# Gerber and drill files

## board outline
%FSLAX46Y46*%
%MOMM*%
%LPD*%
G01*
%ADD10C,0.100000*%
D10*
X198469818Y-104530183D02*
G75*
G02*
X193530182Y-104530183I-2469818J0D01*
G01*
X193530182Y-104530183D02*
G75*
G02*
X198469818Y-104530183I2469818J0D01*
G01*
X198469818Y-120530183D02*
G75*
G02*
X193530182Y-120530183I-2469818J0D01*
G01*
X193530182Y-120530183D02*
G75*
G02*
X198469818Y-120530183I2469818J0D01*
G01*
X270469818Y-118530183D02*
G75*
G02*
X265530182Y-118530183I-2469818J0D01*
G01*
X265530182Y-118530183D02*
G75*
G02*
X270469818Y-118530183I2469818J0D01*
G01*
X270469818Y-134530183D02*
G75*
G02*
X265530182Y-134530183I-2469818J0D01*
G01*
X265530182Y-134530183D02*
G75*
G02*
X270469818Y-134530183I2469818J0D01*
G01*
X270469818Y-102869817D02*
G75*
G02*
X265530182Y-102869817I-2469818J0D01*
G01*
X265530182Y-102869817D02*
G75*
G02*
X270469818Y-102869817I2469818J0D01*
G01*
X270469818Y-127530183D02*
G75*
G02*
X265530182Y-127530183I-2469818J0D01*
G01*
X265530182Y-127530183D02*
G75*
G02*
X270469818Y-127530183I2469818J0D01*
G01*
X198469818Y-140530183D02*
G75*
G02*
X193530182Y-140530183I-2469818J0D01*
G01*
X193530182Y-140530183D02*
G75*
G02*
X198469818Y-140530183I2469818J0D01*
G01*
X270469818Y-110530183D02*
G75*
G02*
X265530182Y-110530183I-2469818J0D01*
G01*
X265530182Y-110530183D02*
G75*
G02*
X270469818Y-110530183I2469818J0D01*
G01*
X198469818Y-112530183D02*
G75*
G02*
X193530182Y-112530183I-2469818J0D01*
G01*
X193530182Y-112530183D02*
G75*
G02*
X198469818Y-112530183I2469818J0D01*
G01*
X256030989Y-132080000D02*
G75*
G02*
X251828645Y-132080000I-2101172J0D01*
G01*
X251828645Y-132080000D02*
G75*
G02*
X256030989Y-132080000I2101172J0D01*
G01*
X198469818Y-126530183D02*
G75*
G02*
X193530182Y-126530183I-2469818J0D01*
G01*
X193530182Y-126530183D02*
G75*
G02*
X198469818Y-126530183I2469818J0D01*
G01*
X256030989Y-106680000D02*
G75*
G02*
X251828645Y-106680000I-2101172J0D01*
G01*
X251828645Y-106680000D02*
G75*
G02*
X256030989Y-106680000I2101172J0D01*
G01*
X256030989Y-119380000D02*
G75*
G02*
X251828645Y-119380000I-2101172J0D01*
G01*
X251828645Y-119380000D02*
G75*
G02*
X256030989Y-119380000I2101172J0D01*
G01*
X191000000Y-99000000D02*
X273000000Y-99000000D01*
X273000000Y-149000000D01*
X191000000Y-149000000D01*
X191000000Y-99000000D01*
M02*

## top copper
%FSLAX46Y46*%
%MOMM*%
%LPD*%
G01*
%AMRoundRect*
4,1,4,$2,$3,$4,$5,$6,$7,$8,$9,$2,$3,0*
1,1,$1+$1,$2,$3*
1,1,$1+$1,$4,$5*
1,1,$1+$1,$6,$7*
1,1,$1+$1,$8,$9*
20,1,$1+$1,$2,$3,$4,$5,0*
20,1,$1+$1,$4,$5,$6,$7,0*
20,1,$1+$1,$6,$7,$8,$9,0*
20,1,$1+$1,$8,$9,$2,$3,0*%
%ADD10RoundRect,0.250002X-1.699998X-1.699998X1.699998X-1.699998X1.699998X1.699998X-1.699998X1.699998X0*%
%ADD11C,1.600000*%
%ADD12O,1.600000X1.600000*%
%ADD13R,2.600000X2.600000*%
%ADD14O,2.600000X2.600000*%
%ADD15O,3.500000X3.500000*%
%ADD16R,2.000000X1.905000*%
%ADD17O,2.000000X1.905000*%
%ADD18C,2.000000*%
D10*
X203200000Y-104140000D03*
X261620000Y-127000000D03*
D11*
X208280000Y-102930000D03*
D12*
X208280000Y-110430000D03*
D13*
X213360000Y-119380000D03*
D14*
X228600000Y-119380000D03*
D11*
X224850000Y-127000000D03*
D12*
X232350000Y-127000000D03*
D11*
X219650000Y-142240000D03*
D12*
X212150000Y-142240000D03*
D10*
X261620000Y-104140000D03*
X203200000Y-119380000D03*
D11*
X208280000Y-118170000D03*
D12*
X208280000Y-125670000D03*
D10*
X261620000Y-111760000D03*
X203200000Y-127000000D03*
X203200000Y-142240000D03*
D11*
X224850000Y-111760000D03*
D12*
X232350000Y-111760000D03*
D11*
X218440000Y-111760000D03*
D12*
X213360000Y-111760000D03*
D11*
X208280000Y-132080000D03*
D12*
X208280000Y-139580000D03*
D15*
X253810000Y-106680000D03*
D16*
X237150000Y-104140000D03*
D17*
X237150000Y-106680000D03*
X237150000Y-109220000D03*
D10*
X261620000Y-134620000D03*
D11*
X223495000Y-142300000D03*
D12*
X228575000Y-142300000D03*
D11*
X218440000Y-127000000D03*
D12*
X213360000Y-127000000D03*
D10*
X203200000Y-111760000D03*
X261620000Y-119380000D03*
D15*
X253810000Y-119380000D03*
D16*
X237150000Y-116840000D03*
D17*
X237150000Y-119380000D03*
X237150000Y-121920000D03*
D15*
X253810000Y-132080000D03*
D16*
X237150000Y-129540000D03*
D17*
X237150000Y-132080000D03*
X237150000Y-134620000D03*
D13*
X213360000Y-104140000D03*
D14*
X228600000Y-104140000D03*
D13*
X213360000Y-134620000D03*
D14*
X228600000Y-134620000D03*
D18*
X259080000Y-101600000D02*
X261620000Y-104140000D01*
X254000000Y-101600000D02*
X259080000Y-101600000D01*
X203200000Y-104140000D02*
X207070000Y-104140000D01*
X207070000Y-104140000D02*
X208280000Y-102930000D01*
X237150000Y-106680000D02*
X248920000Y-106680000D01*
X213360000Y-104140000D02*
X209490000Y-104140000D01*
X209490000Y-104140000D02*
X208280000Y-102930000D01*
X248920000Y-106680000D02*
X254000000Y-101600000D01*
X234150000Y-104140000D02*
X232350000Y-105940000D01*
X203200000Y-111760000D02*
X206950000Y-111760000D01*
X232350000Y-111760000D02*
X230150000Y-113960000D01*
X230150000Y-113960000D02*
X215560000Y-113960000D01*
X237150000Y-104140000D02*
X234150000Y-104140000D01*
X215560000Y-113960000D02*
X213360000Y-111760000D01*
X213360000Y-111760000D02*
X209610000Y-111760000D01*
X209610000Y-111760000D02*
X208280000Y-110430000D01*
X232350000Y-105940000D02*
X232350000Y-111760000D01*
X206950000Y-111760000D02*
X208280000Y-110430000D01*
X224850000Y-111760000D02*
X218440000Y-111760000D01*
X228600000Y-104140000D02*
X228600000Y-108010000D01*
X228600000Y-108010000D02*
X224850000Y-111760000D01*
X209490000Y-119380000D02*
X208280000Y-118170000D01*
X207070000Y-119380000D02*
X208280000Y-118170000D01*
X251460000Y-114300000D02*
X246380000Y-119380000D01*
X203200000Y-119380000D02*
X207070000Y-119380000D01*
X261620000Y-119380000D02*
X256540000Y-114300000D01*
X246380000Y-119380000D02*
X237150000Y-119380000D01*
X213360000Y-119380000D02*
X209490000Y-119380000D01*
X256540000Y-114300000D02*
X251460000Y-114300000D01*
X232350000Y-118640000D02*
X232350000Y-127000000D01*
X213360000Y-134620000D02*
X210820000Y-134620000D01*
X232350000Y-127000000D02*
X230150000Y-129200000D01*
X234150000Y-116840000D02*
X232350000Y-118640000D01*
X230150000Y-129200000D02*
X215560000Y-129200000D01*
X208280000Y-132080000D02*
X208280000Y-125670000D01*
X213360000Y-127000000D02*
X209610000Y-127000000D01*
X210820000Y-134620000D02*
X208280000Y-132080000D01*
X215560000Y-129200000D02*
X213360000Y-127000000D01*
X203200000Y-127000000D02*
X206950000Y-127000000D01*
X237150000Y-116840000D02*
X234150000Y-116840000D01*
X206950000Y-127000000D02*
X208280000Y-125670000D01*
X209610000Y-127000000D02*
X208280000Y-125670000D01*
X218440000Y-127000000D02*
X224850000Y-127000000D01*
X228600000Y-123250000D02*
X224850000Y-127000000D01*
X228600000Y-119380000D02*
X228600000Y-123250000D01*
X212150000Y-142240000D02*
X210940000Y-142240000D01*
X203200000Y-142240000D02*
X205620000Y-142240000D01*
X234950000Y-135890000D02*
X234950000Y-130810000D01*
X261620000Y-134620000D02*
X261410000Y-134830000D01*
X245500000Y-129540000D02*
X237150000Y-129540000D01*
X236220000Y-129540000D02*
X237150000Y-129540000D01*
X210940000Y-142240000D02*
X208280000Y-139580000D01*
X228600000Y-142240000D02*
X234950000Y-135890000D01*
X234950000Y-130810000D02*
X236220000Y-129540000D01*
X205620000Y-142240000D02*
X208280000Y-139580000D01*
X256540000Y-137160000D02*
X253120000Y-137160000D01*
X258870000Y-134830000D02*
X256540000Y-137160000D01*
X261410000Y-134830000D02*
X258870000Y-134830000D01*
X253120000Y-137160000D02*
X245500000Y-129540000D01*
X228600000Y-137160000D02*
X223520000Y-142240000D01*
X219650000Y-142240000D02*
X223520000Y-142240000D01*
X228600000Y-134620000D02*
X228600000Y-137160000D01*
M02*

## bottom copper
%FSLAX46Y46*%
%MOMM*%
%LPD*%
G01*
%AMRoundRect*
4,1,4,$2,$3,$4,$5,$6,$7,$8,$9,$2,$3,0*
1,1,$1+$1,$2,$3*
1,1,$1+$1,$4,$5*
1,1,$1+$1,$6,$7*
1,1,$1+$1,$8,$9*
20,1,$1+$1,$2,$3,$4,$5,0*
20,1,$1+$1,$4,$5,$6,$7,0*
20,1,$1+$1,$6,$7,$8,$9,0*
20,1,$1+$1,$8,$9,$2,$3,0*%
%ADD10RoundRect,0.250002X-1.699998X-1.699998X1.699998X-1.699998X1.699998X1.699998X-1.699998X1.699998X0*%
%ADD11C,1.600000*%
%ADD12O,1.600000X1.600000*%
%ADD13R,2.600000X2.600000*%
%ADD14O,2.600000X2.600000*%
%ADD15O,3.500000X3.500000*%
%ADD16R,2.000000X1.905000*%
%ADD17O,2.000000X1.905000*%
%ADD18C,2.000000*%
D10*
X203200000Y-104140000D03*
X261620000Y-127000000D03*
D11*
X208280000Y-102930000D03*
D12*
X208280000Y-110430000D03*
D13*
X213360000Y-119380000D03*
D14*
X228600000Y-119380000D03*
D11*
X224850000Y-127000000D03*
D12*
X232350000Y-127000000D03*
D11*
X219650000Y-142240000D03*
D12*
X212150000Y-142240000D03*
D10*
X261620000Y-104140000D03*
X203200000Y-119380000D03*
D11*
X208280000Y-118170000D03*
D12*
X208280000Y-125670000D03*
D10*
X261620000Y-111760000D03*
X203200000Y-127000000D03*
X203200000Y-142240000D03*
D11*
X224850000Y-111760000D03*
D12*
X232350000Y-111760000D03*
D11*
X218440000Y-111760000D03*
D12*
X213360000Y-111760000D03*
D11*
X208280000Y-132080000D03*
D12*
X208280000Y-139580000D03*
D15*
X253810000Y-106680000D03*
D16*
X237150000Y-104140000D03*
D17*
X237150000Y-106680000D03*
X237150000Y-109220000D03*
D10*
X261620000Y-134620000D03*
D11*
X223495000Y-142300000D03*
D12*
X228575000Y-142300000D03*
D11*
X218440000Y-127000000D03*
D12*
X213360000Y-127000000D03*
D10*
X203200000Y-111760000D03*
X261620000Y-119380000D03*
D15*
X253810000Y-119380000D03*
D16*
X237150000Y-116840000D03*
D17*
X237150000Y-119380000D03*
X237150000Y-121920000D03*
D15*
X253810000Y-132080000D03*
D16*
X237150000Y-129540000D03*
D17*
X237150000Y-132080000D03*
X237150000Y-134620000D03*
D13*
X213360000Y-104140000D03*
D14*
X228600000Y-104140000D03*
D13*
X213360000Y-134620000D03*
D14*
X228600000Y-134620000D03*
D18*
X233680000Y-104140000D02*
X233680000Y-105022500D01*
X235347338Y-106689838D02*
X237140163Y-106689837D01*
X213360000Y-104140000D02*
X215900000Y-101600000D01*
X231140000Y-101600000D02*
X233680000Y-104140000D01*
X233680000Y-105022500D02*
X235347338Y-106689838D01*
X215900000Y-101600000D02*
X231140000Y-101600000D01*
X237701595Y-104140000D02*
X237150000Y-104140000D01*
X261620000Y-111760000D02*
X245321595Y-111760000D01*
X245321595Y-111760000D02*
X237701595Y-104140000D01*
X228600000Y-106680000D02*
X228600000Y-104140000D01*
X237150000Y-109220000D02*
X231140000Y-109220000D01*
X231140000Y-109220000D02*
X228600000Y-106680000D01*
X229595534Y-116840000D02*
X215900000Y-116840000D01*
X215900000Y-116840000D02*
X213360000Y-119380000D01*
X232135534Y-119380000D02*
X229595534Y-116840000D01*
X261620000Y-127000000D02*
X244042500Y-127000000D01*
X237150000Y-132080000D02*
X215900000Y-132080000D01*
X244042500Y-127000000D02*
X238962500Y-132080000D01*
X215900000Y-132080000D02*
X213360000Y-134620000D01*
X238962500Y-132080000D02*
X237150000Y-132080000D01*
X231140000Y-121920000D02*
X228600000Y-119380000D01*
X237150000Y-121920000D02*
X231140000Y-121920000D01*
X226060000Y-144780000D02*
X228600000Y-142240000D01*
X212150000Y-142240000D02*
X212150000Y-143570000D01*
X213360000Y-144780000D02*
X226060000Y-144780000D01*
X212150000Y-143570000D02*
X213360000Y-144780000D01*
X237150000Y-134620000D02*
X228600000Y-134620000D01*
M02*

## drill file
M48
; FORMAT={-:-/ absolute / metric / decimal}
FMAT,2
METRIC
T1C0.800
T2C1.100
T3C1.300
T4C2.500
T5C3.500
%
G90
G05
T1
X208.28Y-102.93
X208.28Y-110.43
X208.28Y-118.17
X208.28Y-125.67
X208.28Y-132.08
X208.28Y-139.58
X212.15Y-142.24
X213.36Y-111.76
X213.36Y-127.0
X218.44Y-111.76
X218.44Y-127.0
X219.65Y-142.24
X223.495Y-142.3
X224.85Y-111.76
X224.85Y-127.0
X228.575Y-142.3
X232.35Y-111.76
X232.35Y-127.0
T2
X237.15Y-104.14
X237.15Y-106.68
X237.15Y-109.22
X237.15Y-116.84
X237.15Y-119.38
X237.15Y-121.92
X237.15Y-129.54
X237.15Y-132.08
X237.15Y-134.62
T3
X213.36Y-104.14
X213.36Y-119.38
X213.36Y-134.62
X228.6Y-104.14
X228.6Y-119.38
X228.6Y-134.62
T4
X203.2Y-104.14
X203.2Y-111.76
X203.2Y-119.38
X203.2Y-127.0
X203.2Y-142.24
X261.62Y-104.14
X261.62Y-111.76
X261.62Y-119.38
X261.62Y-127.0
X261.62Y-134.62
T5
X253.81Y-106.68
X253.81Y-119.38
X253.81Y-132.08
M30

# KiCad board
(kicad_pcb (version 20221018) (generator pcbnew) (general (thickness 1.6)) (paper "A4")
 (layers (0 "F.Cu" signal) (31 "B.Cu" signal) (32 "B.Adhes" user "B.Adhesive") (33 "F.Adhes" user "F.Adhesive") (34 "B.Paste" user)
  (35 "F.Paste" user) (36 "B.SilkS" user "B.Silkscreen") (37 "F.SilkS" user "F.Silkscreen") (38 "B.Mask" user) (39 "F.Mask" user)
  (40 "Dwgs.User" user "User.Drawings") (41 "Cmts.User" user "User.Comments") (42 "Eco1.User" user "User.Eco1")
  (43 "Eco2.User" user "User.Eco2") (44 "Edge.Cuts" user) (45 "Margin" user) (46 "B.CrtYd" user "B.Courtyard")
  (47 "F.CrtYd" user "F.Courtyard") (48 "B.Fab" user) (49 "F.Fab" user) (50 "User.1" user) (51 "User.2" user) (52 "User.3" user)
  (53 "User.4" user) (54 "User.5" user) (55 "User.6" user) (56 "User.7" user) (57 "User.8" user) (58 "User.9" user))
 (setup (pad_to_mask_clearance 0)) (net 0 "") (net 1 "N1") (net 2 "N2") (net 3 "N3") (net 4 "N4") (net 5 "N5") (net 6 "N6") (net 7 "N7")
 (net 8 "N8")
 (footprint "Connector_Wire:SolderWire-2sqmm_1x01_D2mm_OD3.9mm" (layer "F.Cu") (at 203.2 104.14)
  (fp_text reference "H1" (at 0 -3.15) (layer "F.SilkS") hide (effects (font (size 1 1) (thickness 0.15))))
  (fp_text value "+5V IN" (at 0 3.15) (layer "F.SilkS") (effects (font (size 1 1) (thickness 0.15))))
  (pad "1" thru_hole roundrect (at 0 0) (size 3.9 3.9) (drill 2.5) (layers "*.Cu" "*.Mask") (roundrect_rratio 0.06410307692) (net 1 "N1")))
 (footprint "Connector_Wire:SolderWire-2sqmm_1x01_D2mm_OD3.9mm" (layer "F.Cu") (at 261.62 127)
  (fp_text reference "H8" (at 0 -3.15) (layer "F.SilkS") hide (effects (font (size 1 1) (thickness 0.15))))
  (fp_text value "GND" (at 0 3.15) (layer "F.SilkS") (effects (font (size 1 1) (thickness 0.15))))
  (pad "1" thru_hole roundrect (at 0 0) (size 3.9 3.9) (drill 2.5) (layers "*.Cu" "*.Mask") (roundrect_rratio 0.06410307692) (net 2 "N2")))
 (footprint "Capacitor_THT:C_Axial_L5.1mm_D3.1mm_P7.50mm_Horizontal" (layer "F.Cu") (at 208.28 102.93 -90)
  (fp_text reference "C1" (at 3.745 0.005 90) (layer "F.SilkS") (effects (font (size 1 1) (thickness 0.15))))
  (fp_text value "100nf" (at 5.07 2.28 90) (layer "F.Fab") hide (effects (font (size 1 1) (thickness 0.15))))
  (pad "1" thru_hole circle (at 0 0 270) (size 1.6 1.6) (drill 0.8) (layers "*.Cu" "*.Mask") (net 1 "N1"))
  (pad "2" thru_hole oval (at 7.5 0 270) (size 1.6 1.6) (drill 0.8) (layers "*.Cu" "*.Mask") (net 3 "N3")))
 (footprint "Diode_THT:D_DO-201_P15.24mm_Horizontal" (layer "F.Cu") (at 213.36 119.38)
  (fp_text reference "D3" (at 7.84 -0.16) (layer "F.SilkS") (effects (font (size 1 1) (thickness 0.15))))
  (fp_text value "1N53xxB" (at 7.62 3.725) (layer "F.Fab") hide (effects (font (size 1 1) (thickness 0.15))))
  (pad "1" thru_hole rect (at 0 0) (size 2.6 2.6) (drill 1.3) (layers "*.Cu" "*.Mask") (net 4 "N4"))
  (pad "2" thru_hole oval (at 15.24 0) (size 2.6 2.6) (drill 1.3) (layers "*.Cu" "*.Mask") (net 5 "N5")))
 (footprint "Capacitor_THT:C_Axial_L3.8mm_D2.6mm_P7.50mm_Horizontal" (layer "F.Cu") (at 224.85 127)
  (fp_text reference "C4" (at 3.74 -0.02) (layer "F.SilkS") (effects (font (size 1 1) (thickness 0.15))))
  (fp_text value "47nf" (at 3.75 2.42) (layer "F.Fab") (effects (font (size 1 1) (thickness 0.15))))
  (pad "1" thru_hole circle (at 0 0) (size 1.6 1.6) (drill 0.8) (layers "*.Cu" "*.Mask") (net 5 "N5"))
  (pad "2" thru_hole oval (at 7.5 0) (size 1.6 1.6) (drill 0.8) (layers "*.Cu" "*.Mask") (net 2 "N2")))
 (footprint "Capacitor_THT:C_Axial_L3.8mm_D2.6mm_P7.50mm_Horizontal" (layer "F.Cu") (at 219.65 142.24 180)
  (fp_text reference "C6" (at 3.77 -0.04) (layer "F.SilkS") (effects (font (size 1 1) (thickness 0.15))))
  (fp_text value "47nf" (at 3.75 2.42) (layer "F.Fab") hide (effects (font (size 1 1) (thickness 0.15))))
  (pad "1" thru_hole circle (at 0 0 180) (size 1.6 1.6) (drill 0.8) (layers "*.Cu" "*.Mask") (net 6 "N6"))
  (pad "2" thru_hole oval (at 7.5 0 180) (size 1.6 1.6) (drill 0.8) (layers "*.Cu" "*.Mask") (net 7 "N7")))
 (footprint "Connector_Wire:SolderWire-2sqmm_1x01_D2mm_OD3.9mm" (layer "F.Cu") (at 261.62 104.14)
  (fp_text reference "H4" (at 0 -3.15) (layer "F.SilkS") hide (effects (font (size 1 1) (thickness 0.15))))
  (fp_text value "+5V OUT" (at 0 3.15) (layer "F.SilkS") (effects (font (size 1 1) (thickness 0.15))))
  (pad "1" thru_hole roundrect (at 0 0) (size 3.9 3.9) (drill 2.5) (layers "*.Cu" "*.Mask") (roundrect_rratio 0.06410307692) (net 1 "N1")))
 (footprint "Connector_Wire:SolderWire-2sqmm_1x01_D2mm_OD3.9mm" (layer "F.Cu") (at 203.2 119.38)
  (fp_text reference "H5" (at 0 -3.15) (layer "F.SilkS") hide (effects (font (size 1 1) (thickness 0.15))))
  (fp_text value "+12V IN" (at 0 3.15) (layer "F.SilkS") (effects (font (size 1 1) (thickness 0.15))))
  (pad "1" thru_hole roundrect (at 0 0) (size 3.9 3.9) (drill 2.5) (layers "*.Cu" "*.Mask") (roundrect_rratio 0.06410307692) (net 4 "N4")))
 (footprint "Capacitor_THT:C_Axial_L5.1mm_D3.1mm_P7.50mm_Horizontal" (layer "F.Cu") (at 208.28 118.17 -90)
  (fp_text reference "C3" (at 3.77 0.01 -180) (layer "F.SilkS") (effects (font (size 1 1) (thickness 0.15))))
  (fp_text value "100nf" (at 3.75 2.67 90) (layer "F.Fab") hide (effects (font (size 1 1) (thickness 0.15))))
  (pad "1" thru_hole circle (at 0 0 270) (size 1.6 1.6) (drill 0.8) (layers "*.Cu" "*.Mask") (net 4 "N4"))
  (pad "2" thru_hole oval (at 7.5 0 270) (size 1.6 1.6) (drill 0.8) (layers "*.Cu" "*.Mask") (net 2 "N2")))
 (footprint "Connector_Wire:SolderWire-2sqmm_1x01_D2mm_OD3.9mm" (layer "F.Cu") (at 261.62 111.76)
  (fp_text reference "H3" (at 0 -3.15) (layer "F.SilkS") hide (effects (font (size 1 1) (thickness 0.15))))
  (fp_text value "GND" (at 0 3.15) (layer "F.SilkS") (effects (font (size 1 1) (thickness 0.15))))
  (pad "1" thru_hole roundrect (at 0 0) (size 3.9 3.9) (drill 2.5) (layers "*.Cu" "*.Mask") (roundrect_rratio 0.06410307692) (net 3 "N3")))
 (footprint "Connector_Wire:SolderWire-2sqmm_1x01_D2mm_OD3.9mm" (layer "F.Cu") (at 203.2 127)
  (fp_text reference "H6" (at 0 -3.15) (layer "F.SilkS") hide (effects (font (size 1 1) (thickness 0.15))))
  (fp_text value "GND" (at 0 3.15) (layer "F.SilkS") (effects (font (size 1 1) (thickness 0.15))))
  (pad "1" thru_hole roundrect (at 0 0) (size 3.9 3.9) (drill 2.5) (layers "*.Cu" "*.Mask") (roundrect_rratio 0.06410307692) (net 2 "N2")))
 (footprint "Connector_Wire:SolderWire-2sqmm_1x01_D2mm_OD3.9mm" (layer "F.Cu") (at 203.2 142.24)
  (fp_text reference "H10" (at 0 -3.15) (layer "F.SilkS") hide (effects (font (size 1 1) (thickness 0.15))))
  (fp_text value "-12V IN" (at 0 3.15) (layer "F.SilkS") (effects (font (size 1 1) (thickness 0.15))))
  (pad "1" thru_hole roundrect (at 0 0) (size 3.9 3.9) (drill 2.5) (layers "*.Cu" "*.Mask") (roundrect_rratio 0.06410307692) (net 7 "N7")))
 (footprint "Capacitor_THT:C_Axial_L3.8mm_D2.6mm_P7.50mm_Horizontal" (layer "F.Cu") (at 224.85 111.76)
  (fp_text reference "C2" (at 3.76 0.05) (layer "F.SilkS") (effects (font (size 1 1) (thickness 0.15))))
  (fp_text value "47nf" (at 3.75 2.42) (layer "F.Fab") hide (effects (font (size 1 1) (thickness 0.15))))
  (pad "1" thru_hole circle (at 0 0) (size 1.6 1.6) (drill 0.8) (layers "*.Cu" "*.Mask") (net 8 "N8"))
  (pad "2" thru_hole oval (at 7.5 0) (size 1.6 1.6) (drill 0.8) (layers "*.Cu" "*.Mask") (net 3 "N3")))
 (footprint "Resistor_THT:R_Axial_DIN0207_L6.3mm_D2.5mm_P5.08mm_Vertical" (layer "F.Cu") (at 218.44 111.76 180)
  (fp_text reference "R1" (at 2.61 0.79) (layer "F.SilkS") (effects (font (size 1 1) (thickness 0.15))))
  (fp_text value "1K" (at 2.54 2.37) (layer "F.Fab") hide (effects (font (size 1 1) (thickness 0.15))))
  (pad "1" thru_hole circle (at 0 0 180) (size 1.6 1.6) (drill 0.8) (layers "*.Cu" "*.Mask") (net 8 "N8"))
  (pad "2" thru_hole oval (at 5.08 0 180) (size 1.6 1.6) (drill 0.8) (layers "*.Cu" "*.Mask") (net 3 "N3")))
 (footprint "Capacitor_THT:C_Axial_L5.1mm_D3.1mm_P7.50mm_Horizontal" (layer "F.Cu") (at 208.28 132.08 -90)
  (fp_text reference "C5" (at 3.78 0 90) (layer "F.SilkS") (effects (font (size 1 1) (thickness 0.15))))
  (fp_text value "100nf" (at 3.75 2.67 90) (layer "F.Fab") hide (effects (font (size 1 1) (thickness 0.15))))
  (pad "1" thru_hole circle (at 0 0 270) (size 1.6 1.6) (drill 0.8) (layers "*.Cu" "*.Mask") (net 2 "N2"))
  (pad "2" thru_hole oval (at 7.5 0 270) (size 1.6 1.6) (drill 0.8) (layers "*.Cu" "*.Mask") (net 7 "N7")))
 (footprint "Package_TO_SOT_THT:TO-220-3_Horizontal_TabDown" (layer "F.Cu") (at 237.15 104.14 -90)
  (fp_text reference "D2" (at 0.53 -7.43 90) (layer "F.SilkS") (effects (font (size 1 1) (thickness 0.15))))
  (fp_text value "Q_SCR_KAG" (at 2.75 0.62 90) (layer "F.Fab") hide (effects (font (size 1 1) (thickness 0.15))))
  (pad "" thru_hole oval (at 2.54 -16.66 270) (size 3.5 3.5) (drill 3.5) (layers "*.Cu" "*.Mask"))
  (pad "1" thru_hole rect (at 0 0 270) (size 1.905 2) (drill 1.1) (layers "*.Cu" "*.Mask") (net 3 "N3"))
  (pad "2" thru_hole oval (at 2.54 0 270) (size 1.905 2) (drill 1.1) (layers "*.Cu" "*.Mask") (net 1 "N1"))
  (pad "3" thru_hole oval (at 5.08 0 270) (size 1.905 2) (drill 1.1) (layers "*.Cu" "*.Mask") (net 8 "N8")))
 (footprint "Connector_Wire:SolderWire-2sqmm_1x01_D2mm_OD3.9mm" (layer "F.Cu") (at 261.62 134.62)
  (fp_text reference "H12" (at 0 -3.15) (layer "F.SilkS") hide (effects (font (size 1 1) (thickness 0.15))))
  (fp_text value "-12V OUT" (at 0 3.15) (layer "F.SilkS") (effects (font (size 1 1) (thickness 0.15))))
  (pad "1" thru_hole roundrect (at 0 0) (size 3.9 3.9) (drill 2.5) (layers "*.Cu" "*.Mask") (roundrect_rratio 0.06410307692) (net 7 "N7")))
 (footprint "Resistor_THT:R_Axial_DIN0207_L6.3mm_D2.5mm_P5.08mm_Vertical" (layer "F.Cu") (at 223.495 142.3)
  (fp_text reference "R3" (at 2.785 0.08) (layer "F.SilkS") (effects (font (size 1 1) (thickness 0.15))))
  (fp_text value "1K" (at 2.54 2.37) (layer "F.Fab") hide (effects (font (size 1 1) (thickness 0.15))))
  (pad "1" thru_hole circle (at 0 0) (size 1.6 1.6) (drill 0.8) (layers "*.Cu" "*.Mask") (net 6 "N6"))
  (pad "2" thru_hole oval (at 5.08 0) (size 1.6 1.6) (drill 0.8) (layers "*.Cu" "*.Mask") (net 7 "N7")))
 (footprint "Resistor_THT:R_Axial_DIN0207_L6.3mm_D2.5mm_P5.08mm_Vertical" (layer "F.Cu") (at 218.44 127 180)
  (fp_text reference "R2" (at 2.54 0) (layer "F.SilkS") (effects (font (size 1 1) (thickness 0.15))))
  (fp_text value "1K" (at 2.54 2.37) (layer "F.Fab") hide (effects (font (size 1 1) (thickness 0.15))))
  (pad "1" thru_hole circle (at 0 0 180) (size 1.6 1.6) (drill 0.8) (layers "*.Cu" "*.Mask") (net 5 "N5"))
  (pad "2" thru_hole oval (at 5.08 0 180) (size 1.6 1.6) (drill 0.8) (layers "*.Cu" "*.Mask") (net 2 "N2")))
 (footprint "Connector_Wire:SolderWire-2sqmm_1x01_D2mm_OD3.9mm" (layer "F.Cu") (at 203.2 111.76)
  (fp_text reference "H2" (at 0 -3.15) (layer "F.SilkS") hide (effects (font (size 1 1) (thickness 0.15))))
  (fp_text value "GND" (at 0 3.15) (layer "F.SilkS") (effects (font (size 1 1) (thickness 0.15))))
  (pad "1" thru_hole roundrect (at 0 0) (size 3.9 3.9) (drill 2.5) (layers "*.Cu" "*.Mask") (roundrect_rratio 0.06410307692) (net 3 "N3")))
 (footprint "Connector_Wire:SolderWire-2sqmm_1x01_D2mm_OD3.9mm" (layer "F.Cu") (at 261.62 119.38)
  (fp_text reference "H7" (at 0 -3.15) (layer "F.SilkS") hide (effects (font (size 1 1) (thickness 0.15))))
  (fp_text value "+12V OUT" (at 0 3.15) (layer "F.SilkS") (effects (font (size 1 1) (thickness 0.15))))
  (pad "1" thru_hole roundrect (at 0 0) (size 3.9 3.9) (drill 2.5) (layers "*.Cu" "*.Mask") (roundrect_rratio 0.06410307692) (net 4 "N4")))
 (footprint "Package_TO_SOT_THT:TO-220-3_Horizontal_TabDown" (layer "F.Cu") (at 237.15 116.84 -90)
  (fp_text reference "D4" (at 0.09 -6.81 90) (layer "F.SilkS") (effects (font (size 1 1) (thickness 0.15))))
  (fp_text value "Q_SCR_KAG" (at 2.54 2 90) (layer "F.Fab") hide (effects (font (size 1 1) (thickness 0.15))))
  (pad "" thru_hole oval (at 2.54 -16.66 270) (size 3.5 3.5) (drill 3.5) (layers "*.Cu" "*.Mask"))
  (pad "1" thru_hole rect (at 0 0 270) (size 1.905 2) (drill 1.1) (layers "*.Cu" "*.Mask") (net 2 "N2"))
  (pad "2" thru_hole oval (at 2.54 0 270) (size 1.905 2) (drill 1.1) (layers "*.Cu" "*.Mask") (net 4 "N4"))
  (pad "3" thru_hole oval (at 5.08 0 270) (size 1.905 2) (drill 1.1) (layers "*.Cu" "*.Mask") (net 5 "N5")))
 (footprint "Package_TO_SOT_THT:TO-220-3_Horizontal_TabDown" (layer "F.Cu") (at 237.15 129.54 -90)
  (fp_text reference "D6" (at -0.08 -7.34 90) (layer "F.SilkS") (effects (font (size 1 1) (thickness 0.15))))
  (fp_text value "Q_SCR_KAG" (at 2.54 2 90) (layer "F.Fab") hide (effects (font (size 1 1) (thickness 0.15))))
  (pad "" thru_hole oval (at 2.54 -16.66 270) (size 3.5 3.5) (drill 3.5) (layers "*.Cu" "*.Mask"))
  (pad "1" thru_hole rect (at 0 0 270) (size 1.905 2) (drill 1.1) (layers "*.Cu" "*.Mask") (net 7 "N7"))
  (pad "2" thru_hole oval (at 2.54 0 270) (size 1.905 2) (drill 1.1) (layers "*.Cu" "*.Mask") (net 2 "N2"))
  (pad "3" thru_hole oval (at 5.08 0 270) (size 1.905 2) (drill 1.1) (layers "*.Cu" "*.Mask") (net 6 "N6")))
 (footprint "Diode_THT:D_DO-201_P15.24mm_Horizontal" (layer "F.Cu") (at 213.36 104.14)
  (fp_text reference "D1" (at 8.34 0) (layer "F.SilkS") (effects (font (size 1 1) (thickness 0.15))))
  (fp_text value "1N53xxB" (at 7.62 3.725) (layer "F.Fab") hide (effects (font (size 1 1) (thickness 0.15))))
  (pad "1" thru_hole rect (at 0 0) (size 2.6 2.6) (drill 1.3) (layers "*.Cu" "*.Mask") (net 1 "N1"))
  (pad "2" thru_hole oval (at 15.24 0) (size 2.6 2.6) (drill 1.3) (layers "*.Cu" "*.Mask") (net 8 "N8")))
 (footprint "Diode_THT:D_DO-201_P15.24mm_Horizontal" (layer "F.Cu") (at 213.36 134.62)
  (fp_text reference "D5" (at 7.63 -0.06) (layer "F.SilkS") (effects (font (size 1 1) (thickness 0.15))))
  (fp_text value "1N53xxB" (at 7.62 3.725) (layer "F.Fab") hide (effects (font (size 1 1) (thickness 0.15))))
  (pad "1" thru_hole rect (at 0 0) (size 2.6 2.6) (drill 1.3) (layers "*.Cu" "*.Mask") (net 2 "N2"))
  (pad "2" thru_hole oval (at 15.24 0) (size 2.6 2.6) (drill 1.3) (layers "*.Cu" "*.Mask") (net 6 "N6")))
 (gr_circle (center 196 104.530183) (end 197.3 106.630183) (stroke (width 0.1) (type default)) (fill none) (layer "Edge.Cuts"))
 (gr_circle (center 196 120.530183) (end 197.3 122.630183) (stroke (width 0.1) (type default)) (fill none) (layer "Edge.Cuts"))
 (gr_circle (center 268 118.530183) (end 269.3 120.630183) (stroke (width 0.1) (type default)) (fill none) (layer "Edge.Cuts"))
 (gr_circle (center 268 134.530183) (end 269.3 136.630183) (stroke (width 0.1) (type default)) (fill none) (layer "Edge.Cuts"))
 (gr_circle (center 268 102.869817) (end 269.3 104.969817) (stroke (width 0.1) (type default)) (fill none) (layer "Edge.Cuts"))
 (gr_circle (center 268 127.530183) (end 269.3 129.630183) (stroke (width 0.1) (type default)) (fill none) (layer "Edge.Cuts"))
 (gr_circle (center 196 140.530183) (end 197.3 142.630183) (stroke (width 0.1) (type default)) (fill none) (layer "Edge.Cuts"))
 (gr_circle (center 268 110.530183) (end 269.3 112.630183) (stroke (width 0.1) (type default)) (fill none) (layer "Edge.Cuts"))
 (gr_circle (center 196 112.530183) (end 197.3 114.630183) (stroke (width 0.1) (type default)) (fill none) (layer "Edge.Cuts"))
 (gr_circle (center 253.929817 132.08) (end 254 134.18) (stroke (width 0.1) (type default)) (fill none) (layer "Edge.Cuts"))
 (gr_circle (center 196 126.530183) (end 197.3 128.630183) (stroke (width 0.1) (type default)) (fill none) (layer "Edge.Cuts"))
 (gr_circle (center 253.929817 106.68) (end 254 108.78) (stroke (width 0.1) (type default)) (fill none) (layer "Edge.Cuts"))
 (gr_circle (center 253.929817 119.38) (end 254 121.48) (stroke (width 0.1) (type default)) (fill none) (layer "Edge.Cuts"))
 (gr_rect (start 191 99) (end 273 149) (stroke (width 0.1) (type default)) (fill none) (layer "Edge.Cuts"))
 (segment (start 259.08 101.6) (end 261.62 104.14) (width 2) (layer "F.Cu") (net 1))
 (segment (start 254 101.6) (end 259.08 101.6) (width 2) (layer "F.Cu") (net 1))
 (segment (start 203.2 104.14) (end 207.07 104.14) (width 2) (layer "F.Cu") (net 1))
 (segment (start 207.07 104.14) (end 208.28 102.93) (width 2) (layer "F.Cu") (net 1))
 (segment (start 237.15 106.68) (end 248.92 106.68) (width 2) (layer "F.Cu") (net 1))
 (segment (start 213.36 104.14) (end 209.49 104.14) (width 2) (layer "F.Cu") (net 1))
 (segment (start 209.49 104.14) (end 208.28 102.93) (width 2) (layer "F.Cu") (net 1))
 (segment (start 248.92 106.68) (end 254 101.6) (width 2) (layer "F.Cu") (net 1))
 (segment (start 233.68 104.14) (end 233.68 105.0225) (width 2) (layer "B.Cu") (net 1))
 (segment (start 235.347338 106.689838) (end 237.140163 106.689837) (width 2) (layer "B.Cu") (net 1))
 (segment (start 213.36 104.14) (end 215.9 101.6) (width 2) (layer "B.Cu") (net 1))
 (segment (start 231.14 101.6) (end 233.68 104.14) (width 2) (layer "B.Cu") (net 1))
 (segment (start 233.68 105.0225) (end 235.347338 106.689838) (width 2) (layer "B.Cu") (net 1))
 (segment (start 215.9 101.6) (end 231.14 101.6) (width 2) (layer "B.Cu") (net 1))
 (segment (start 234.15 104.14) (end 232.35 105.94) (width 2) (layer "F.Cu") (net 3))
 (segment (start 203.2 111.76) (end 206.95 111.76) (width 2) (layer "F.Cu") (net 3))
 (segment (start 232.35 111.76) (end 230.15 113.96) (width 2) (layer "F.Cu") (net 3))
 (segment (start 230.15 113.96) (end 215.56 113.96) (width 2) (layer "F.Cu") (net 3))
 (segment (start 237.15 104.14) (end 234.15 104.14) (width 2) (layer "F.Cu") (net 3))
 (segment (start 215.56 113.96) (end 213.36 111.76) (width 2) (layer "F.Cu") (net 3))
 (segment (start 213.36 111.76) (end 209.61 111.76) (width 2) (layer "F.Cu") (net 3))
 (segment (start 209.61 111.76) (end 208.28 110.43) (width 2) (layer "F.Cu") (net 3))
 (segment (start 232.35 105.94) (end 232.35 111.76) (width 2) (layer "F.Cu") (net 3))
 (segment (start 206.95 111.76) (end 208.28 110.43) (width 2) (layer "F.Cu") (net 3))
 (segment (start 237.701595 104.14) (end 237.15 104.14) (width 2) (layer "B.Cu") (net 3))
 (segment (start 261.62 111.76) (end 245.321595 111.76) (width 2) (layer "B.Cu") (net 3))
 (segment (start 245.321595 111.76) (end 237.701595 104.14) (width 2) (layer "B.Cu") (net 3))
 (segment (start 224.85 111.76) (end 218.44 111.76) (width 2) (layer "F.Cu") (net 8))
 (segment (start 228.6 104.14) (end 228.6 108.01) (width 2) (layer "F.Cu") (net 8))
 (segment (start 228.6 108.01) (end 224.85 111.76) (width 2) (layer "F.Cu") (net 8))
 (segment (start 228.6 106.68) (end 228.6 104.14) (width 2) (layer "B.Cu") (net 8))
 (segment (start 237.15 109.22) (end 231.14 109.22) (width 2) (layer "B.Cu") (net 8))
 (segment (start 231.14 109.22) (end 228.6 106.68) (width 2) (layer "B.Cu") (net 8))
 (segment (start 209.49 119.38) (end 208.28 118.17) (width 2) (layer "F.Cu") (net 4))
 (segment (start 207.07 119.38) (end 208.28 118.17) (width 2) (layer "F.Cu") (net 4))
 (segment (start 251.46 114.3) (end 246.38 119.38) (width 2) (layer "F.Cu") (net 4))
 (segment (start 203.2 119.38) (end 207.07 119.38) (width 2) (layer "F.Cu") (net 4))
 (segment (start 261.62 119.38) (end 256.54 114.3) (width 2) (layer "F.Cu") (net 4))
 (segment (start 246.38 119.38) (end 237.15 119.38) (width 2) (layer "F.Cu") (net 4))
 (segment (start 213.36 119.38) (end 209.49 119.38) (width 2) (layer "F.Cu") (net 4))
 (segment (start 256.54 114.3) (end 251.46 114.3) (width 2) (layer "F.Cu") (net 4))
 (segment (start 229.595534 116.84) (end 215.9 116.84) (width 2) (layer "B.Cu") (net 4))
 (segment (start 215.9 116.84) (end 213.36 119.38) (width 2) (layer "B.Cu") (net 4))
 (segment (start 232.135534 119.38) (end 229.595534 116.84) (width 2) (layer "B.Cu") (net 4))
 (segment (start 232.35 118.64) (end 232.35 127) (width 2) (layer "F.Cu") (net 2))
 (segment (start 213.36 134.62) (end 210.82 134.62) (width 2) (layer "F.Cu") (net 2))
 (segment (start 232.35 127) (end 230.15 129.2) (width 2) (layer "F.Cu") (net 2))
 (segment (start 234.15 116.84) (end 232.35 118.64) (width 2) (layer "F.Cu") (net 2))
 (segment (start 230.15 129.2) (end 215.56 129.2) (width 2) (layer "F.Cu") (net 2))
 (segment (start 208.28 132.08) (end 208.28 125.67) (width 2) (layer "F.Cu") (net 2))
 (segment (start 213.36 127) (end 209.61 127) (width 2) (layer "F.Cu") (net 2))
 (segment (start 210.82 134.62) (end 208.28 132.08) (width 2) (layer "F.Cu") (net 2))
 (segment (start 215.56 129.2) (end 213.36 127) (width 2) (layer "F.Cu") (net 2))
 (segment (start 203.2 127) (end 206.95 127) (width 2) (layer "F.Cu") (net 2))
 (segment (start 237.15 116.84) (end 234.15 116.84) (width 2) (layer "F.Cu") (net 2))
 (segment (start 206.95 127) (end 208.28 125.67) (width 2) (layer "F.Cu") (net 2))
 (segment (start 209.61 127) (end 208.28 125.67) (width 2) (layer "F.Cu") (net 2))
 (segment (start 261.62 127) (end 244.0425 127) (width 2) (layer "B.Cu") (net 2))
 (segment (start 237.15 132.08) (end 215.9 132.08) (width 2) (layer "B.Cu") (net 2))
 (segment (start 244.0425 127) (end 238.9625 132.08) (width 2) (layer "B.Cu") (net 2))
 (segment (start 215.9 132.08) (end 213.36 134.62) (width 2) (layer "B.Cu") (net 2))
 (segment (start 238.9625 132.08) (end 237.15 132.08) (width 2) (layer "B.Cu") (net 2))
 (segment (start 218.44 127) (end 224.85 127) (width 2) (layer "F.Cu") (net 5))
 (segment (start 228.6 123.25) (end 224.85 127) (width 2) (layer "F.Cu") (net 5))
 (segment (start 228.6 119.38) (end 228.6 123.25) (width 2) (layer "F.Cu") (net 5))
 (segment (start 231.14 121.92) (end 228.6 119.38) (width 2) (layer "B.Cu") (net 5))
 (segment (start 237.15 121.92) (end 231.14 121.92) (width 2) (layer "B.Cu") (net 5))
 (segment (start 212.15 142.24) (end 210.94 142.24) (width 2) (layer "F.Cu") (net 7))
 (segment (start 203.2 142.24) (end 205.62 142.24) (width 2) (layer "F.Cu") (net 7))
 (segment (start 234.95 135.89) (end 234.95 130.81) (width 2) (layer "F.Cu") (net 7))
 (segment (start 261.62 134.62) (end 261.41 134.83) (width 2) (layer "F.Cu") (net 7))
 (segment (start 245.5 129.54) (end 237.15 129.54) (width 2) (layer "F.Cu") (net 7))
 (segment (start 236.22 129.54) (end 237.15 129.54) (width 2) (layer "F.Cu") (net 7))
 (segment (start 210.94 142.24) (end 208.28 139.58) (width 2) (layer "F.Cu") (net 7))
 (segment (start 228.6 142.24) (end 234.95 135.89) (width 2) (layer "F.Cu") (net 7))
 (segment (start 234.95 130.81) (end 236.22 129.54) (width 2) (layer "F.Cu") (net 7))
 (segment (start 205.62 142.24) (end 208.28 139.58) (width 2) (layer "F.Cu") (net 7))
 (segment (start 256.54 137.16) (end 253.12 137.16) (width 2) (layer "F.Cu") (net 7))
 (segment (start 258.87 134.83) (end 256.54 137.16) (width 2) (layer "F.Cu") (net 7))
 (segment (start 261.41 134.83) (end 258.87 134.83) (width 2) (layer "F.Cu") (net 7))
 (segment (start 253.12 137.16) (end 245.5 129.54) (width 2) (layer "F.Cu") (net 7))
 (segment (start 226.06 144.78) (end 228.6 142.24) (width 2) (layer "B.Cu") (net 7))
 (segment (start 212.15 142.24) (end 212.15 143.57) (width 2) (layer "B.Cu") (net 7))
 (segment (start 213.36 144.78) (end 226.06 144.78) (width 2) (layer "B.Cu") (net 7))
 (segment (start 212.15 143.57) (end 213.36 144.78) (width 2) (layer "B.Cu") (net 7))
 (segment (start 228.6 137.16) (end 223.52 142.24) (width 2) (layer "F.Cu") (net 6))
 (segment (start 219.65 142.24) (end 223.52 142.24) (width 2) (layer "F.Cu") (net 6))
 (segment (start 228.6 134.62) (end 228.6 137.16) (width 2) (layer "F.Cu") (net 6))
 (segment (start 237.15 134.62) (end 228.6 134.62) (width 2) (layer "B.Cu") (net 6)))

